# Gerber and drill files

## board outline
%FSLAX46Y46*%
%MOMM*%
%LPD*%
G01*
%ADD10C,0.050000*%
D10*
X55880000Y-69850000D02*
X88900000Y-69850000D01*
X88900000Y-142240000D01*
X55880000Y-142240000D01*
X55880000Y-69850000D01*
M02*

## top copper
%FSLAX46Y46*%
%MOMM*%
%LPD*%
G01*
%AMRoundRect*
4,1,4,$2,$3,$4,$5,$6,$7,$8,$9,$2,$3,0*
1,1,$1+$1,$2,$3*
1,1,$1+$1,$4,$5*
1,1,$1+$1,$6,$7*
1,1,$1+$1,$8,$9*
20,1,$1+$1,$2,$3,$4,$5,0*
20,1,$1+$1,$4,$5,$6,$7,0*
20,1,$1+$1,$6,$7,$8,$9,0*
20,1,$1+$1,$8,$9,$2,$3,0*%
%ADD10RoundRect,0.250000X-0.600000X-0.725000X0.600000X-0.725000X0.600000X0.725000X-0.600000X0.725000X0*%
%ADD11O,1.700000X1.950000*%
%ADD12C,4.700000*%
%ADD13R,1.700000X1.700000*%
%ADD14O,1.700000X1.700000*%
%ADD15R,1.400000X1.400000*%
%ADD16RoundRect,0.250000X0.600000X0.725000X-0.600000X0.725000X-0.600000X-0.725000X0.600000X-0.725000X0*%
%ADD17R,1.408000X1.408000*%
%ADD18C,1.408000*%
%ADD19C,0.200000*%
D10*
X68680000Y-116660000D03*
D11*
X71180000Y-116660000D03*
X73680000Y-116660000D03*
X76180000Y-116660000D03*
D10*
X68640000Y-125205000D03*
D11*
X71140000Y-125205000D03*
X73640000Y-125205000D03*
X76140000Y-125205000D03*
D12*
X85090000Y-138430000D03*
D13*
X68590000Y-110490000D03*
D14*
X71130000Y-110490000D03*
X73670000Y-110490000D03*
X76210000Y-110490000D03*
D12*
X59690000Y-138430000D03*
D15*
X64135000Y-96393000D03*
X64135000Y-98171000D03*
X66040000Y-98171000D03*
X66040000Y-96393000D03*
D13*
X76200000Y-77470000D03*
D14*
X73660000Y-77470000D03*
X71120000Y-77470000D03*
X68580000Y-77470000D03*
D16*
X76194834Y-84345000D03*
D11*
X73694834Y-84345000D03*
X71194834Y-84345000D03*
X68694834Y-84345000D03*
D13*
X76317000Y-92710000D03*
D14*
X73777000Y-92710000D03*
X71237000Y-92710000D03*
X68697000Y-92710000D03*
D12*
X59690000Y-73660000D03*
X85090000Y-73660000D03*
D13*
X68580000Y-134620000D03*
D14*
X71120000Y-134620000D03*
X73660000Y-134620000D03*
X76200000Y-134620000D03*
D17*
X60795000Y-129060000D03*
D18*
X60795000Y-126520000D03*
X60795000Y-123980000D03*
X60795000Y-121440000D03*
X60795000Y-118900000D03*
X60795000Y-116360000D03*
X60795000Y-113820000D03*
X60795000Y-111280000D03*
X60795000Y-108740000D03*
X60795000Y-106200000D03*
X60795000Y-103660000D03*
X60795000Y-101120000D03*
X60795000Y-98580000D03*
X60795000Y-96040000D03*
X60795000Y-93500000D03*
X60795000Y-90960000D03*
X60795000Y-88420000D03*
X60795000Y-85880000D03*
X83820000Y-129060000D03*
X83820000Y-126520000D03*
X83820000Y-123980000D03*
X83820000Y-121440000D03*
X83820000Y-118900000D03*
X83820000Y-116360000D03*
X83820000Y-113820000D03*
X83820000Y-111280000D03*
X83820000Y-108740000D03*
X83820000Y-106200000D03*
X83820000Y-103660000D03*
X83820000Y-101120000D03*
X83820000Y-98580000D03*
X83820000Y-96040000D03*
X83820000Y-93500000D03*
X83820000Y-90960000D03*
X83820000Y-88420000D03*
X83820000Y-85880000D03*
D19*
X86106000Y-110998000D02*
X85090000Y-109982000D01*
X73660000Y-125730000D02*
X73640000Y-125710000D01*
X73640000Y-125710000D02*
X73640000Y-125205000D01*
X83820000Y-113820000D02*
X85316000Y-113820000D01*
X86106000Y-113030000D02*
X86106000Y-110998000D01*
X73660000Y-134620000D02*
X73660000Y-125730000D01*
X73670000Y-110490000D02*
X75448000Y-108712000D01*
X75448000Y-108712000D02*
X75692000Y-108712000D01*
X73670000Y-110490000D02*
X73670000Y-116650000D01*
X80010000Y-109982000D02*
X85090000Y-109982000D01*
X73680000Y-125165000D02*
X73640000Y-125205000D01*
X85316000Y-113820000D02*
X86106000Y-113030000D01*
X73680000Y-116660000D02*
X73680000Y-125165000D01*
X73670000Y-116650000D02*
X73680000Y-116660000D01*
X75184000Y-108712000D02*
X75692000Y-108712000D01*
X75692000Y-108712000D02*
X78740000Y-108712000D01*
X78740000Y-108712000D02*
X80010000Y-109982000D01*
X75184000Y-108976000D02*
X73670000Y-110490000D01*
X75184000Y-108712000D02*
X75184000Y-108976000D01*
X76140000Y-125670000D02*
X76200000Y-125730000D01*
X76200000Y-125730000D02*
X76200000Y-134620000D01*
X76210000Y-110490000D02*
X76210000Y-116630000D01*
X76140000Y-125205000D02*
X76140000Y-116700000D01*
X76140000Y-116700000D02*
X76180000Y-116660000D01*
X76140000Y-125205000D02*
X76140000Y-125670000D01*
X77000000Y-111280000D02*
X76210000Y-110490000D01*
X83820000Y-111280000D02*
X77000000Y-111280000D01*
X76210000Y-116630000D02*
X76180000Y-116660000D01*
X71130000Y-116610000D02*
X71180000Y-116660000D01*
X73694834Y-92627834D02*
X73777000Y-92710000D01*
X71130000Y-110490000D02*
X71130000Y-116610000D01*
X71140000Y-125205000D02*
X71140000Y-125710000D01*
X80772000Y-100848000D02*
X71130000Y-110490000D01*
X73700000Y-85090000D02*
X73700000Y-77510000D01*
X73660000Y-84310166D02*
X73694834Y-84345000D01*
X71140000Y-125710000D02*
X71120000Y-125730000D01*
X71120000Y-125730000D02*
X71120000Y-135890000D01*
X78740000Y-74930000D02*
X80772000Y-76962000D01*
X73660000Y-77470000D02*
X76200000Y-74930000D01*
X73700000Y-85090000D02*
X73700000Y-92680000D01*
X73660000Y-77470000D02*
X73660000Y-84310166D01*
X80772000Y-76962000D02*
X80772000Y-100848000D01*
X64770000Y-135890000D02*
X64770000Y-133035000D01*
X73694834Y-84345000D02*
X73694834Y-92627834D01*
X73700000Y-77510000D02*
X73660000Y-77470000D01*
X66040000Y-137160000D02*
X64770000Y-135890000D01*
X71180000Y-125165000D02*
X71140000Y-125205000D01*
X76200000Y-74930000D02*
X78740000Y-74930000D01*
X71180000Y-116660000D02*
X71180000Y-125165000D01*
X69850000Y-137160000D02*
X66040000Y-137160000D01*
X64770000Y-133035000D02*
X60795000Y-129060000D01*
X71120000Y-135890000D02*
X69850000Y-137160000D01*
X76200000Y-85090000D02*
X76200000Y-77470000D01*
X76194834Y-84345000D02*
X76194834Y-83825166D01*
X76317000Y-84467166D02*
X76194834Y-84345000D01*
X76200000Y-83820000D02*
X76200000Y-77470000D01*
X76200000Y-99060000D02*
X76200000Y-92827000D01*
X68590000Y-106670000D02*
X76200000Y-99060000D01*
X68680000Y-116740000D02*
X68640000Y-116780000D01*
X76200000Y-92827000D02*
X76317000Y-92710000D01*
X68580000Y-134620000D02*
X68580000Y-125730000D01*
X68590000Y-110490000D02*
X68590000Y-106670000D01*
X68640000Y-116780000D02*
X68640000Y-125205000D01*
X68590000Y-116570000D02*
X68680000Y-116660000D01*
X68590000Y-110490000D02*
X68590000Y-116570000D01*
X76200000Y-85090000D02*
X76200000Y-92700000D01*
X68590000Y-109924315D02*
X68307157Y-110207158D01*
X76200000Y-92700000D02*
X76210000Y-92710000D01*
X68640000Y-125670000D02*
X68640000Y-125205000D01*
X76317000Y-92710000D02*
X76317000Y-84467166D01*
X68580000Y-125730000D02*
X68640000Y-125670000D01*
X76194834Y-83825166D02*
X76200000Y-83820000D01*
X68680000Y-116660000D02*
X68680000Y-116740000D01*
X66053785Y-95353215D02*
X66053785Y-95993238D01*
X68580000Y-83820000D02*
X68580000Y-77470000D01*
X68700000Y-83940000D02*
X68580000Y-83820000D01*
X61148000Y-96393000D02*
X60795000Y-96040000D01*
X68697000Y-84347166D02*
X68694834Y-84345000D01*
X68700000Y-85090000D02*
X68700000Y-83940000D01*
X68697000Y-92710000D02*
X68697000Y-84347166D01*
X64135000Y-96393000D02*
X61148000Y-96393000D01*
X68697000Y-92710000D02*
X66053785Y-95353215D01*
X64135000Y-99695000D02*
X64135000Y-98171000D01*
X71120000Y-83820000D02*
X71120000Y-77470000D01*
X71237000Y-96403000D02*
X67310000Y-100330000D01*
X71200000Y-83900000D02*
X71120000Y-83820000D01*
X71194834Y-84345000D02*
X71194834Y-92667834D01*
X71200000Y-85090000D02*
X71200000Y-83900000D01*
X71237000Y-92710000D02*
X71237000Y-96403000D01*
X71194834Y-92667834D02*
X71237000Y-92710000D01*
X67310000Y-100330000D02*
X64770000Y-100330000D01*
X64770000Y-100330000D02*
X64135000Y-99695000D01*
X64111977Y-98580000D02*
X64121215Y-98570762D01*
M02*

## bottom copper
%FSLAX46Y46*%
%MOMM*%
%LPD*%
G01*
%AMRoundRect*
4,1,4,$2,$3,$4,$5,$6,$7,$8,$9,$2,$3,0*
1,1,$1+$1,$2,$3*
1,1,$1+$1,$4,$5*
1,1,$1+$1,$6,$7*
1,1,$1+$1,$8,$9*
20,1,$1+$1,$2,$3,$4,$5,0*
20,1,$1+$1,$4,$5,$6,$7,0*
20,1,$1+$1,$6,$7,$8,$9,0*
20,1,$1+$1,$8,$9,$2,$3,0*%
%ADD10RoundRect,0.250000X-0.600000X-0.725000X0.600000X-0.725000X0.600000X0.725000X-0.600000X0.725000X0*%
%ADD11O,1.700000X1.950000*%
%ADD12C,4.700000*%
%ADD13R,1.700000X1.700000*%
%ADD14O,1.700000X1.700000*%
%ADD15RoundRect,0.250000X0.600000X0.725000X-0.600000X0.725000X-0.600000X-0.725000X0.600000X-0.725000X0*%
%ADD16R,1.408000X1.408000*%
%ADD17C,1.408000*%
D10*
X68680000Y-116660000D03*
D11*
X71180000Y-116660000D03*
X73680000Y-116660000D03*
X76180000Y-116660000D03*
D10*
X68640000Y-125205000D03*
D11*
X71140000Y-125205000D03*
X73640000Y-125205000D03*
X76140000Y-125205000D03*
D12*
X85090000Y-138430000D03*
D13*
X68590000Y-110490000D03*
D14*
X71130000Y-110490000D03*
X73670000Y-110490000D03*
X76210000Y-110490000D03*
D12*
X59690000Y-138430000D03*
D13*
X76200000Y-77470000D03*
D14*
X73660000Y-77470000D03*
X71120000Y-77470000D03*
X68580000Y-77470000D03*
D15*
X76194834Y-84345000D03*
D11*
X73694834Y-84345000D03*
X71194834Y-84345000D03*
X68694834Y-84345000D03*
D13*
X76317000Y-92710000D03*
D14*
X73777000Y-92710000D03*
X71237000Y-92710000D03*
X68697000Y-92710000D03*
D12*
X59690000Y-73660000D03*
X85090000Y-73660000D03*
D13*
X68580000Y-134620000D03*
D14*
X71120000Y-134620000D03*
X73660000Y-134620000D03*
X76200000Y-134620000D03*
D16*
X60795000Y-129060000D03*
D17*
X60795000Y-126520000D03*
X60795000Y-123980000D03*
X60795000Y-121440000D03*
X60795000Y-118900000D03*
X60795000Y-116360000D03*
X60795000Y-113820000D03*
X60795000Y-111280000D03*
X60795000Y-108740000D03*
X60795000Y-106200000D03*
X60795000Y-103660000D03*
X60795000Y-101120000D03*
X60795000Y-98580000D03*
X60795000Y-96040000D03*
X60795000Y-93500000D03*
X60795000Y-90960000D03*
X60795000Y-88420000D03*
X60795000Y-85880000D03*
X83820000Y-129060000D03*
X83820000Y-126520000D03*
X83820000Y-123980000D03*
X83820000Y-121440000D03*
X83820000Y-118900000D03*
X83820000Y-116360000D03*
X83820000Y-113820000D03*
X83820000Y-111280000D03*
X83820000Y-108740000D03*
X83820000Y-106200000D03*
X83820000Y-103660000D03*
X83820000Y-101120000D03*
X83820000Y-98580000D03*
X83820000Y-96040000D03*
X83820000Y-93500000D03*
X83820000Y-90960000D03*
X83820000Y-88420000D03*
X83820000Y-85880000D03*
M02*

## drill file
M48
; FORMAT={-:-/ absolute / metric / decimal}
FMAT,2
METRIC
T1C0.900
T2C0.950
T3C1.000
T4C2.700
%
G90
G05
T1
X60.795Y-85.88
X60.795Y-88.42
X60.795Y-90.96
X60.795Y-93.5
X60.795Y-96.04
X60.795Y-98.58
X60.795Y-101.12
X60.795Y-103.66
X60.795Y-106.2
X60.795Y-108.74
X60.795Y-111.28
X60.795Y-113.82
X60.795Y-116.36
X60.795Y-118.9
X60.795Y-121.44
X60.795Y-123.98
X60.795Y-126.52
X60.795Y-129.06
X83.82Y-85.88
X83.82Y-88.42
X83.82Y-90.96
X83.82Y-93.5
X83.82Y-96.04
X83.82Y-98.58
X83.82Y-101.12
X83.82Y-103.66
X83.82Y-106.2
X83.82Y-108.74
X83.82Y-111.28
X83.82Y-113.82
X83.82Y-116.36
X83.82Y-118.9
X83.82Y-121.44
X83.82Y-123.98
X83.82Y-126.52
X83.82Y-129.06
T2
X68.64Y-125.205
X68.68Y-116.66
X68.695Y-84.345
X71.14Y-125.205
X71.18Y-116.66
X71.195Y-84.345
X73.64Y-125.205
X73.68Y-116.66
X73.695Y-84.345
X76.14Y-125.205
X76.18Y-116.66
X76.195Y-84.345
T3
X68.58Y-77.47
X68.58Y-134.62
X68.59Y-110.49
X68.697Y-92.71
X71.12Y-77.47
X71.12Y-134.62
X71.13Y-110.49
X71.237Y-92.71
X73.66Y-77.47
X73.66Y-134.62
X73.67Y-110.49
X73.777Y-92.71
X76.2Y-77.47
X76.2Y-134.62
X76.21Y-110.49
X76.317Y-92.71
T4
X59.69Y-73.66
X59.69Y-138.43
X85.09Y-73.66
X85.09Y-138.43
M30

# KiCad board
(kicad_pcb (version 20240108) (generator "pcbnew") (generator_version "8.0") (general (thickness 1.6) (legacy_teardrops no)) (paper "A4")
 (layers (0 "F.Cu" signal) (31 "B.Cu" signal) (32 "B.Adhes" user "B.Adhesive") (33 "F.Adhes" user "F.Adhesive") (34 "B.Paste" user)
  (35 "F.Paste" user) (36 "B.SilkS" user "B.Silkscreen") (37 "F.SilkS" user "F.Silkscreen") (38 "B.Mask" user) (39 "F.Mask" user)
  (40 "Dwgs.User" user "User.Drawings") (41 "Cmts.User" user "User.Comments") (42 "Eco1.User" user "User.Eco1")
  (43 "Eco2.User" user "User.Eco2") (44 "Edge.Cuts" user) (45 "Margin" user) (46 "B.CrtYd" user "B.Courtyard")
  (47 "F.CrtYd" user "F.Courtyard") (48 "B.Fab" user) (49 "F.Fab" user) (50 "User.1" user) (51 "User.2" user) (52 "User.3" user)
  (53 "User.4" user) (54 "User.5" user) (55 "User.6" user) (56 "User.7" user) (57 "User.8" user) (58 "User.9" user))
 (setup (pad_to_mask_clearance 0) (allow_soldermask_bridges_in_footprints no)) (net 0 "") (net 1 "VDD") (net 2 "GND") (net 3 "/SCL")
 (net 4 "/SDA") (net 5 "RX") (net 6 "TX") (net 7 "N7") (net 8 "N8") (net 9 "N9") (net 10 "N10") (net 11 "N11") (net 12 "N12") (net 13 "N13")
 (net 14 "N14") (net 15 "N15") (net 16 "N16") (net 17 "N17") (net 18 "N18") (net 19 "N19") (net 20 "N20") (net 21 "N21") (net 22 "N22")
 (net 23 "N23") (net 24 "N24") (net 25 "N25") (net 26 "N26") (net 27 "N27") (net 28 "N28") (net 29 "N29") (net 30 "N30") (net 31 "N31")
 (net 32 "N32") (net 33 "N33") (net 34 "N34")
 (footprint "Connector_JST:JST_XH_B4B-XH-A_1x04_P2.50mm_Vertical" (layer "F.Cu") (at 68.68 116.66)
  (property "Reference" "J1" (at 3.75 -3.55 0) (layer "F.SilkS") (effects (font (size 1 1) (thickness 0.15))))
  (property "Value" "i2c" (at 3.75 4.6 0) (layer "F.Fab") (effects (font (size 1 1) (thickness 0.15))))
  (pad "1" thru_hole roundrect (at 0 0) (size 1.7 1.95) (drill 0.95) (layers "*.Cu" "*.Mask") (remove_unused_layers no)
   (roundrect_rratio 0.147059) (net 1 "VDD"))
  (pad "2" thru_hole oval (at 2.5 0) (size 1.7 1.95) (drill 0.95) (layers "*.Cu" "*.Mask") (remove_unused_layers no) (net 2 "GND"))
  (pad "3" thru_hole oval (at 5 0) (size 1.7 1.95) (drill 0.95) (layers "*.Cu" "*.Mask") (remove_unused_layers no) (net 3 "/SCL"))
  (pad "4" thru_hole oval (at 7.5 0) (size 1.7 1.95) (drill 0.95) (layers "*.Cu" "*.Mask") (remove_unused_layers no) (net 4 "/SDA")))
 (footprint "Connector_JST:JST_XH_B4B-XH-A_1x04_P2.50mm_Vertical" (layer "F.Cu") (at 68.64 125.205)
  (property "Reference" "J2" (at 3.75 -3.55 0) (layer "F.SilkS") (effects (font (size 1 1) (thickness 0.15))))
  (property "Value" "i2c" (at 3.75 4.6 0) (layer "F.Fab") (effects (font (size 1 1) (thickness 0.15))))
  (pad "1" thru_hole roundrect (at 0 0) (size 1.7 1.95) (drill 0.95) (layers "*.Cu" "*.Mask") (remove_unused_layers no)
   (roundrect_rratio 0.147059) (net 1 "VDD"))
  (pad "2" thru_hole oval (at 2.5 0) (size 1.7 1.95) (drill 0.95) (layers "*.Cu" "*.Mask") (remove_unused_layers no) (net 2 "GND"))
  (pad "3" thru_hole oval (at 5 0) (size 1.7 1.95) (drill 0.95) (layers "*.Cu" "*.Mask") (remove_unused_layers no) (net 3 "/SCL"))
  (pad "4" thru_hole oval (at 7.5 0) (size 1.7 1.95) (drill 0.95) (layers "*.Cu" "*.Mask") (remove_unused_layers no) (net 4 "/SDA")))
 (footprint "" (layer "F.Cu") (at 85.09 138.43)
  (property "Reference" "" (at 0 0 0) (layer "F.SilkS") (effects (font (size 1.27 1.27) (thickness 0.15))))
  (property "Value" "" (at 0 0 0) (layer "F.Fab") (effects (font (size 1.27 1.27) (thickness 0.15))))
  (pad "1" thru_hole circle (at 0 0) (size 4.7 4.7) (drill 2.7) (layers "*.Cu" "*.Mask") (remove_unused_layers no)))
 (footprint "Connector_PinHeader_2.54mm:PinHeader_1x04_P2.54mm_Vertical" (layer "F.Cu") (at 68.59 110.49 90)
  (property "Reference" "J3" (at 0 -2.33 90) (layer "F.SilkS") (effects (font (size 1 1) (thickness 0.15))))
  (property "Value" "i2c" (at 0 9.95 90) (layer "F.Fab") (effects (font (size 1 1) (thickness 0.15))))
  (pad "1" thru_hole rect (at 0 0 90) (size 1.7 1.7) (drill 1) (layers "*.Cu" "*.Mask") (remove_unused_layers no) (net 1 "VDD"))
  (pad "2" thru_hole oval (at 0 2.54 90) (size 1.7 1.7) (drill 1) (layers "*.Cu" "*.Mask") (remove_unused_layers no) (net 2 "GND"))
  (pad "3" thru_hole oval (at 0 5.08 90) (size 1.7 1.7) (drill 1) (layers "*.Cu" "*.Mask") (remove_unused_layers no) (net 3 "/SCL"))
  (pad "4" thru_hole oval (at 0 7.62 90) (size 1.7 1.7) (drill 1) (layers "*.Cu" "*.Mask") (remove_unused_layers no) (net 4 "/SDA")))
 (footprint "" (layer "F.Cu") (at 59.69 138.43)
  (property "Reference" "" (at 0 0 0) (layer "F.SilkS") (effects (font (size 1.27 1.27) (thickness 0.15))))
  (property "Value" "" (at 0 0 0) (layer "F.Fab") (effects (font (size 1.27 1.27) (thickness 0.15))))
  (pad "1" thru_hole circle (at 0 0) (size 4.7 4.7) (drill 2.7) (layers "*.Cu" "*.Mask") (remove_unused_layers no)))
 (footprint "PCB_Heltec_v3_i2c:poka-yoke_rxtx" (layer "F.Cu") (at 65.024 94.742)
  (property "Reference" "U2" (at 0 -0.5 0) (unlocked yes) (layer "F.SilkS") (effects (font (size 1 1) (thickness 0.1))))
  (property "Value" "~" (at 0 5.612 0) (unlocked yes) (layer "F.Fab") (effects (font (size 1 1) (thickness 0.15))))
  (pad "1" smd rect (at -0.889 1.651) (size 1.4 1.4) (layers "F.Cu" "F.Paste" "F.Mask") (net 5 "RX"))
  (pad "2" smd rect (at -0.889 3.429) (size 1.4 1.4) (layers "F.Cu" "F.Paste" "F.Mask") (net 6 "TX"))
  (pad "3" smd rect (at 1.016 3.429) (size 1.4 1.4) (layers "F.Cu" "F.Paste" "F.Mask") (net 6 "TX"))
  (pad "4" smd rect (at 1.016 1.651) (size 1.4 1.4) (layers "F.Cu" "F.Paste" "F.Mask") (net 5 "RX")))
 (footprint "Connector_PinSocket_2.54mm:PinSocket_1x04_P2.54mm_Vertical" (layer "F.Cu") (at 76.2 77.47 -90)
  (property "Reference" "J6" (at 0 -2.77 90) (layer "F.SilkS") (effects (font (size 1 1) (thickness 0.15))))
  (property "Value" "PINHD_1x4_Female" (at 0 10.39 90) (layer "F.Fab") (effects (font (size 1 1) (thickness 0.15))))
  (pad "1" thru_hole rect (at 0 0 270) (size 1.7 1.7) (drill 1) (layers "*.Cu" "*.Mask") (remove_unused_layers no) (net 1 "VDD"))
  (pad "2" thru_hole oval (at 0 2.54 270) (size 1.7 1.7) (drill 1) (layers "*.Cu" "*.Mask") (remove_unused_layers no) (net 2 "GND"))
  (pad "3" thru_hole oval (at 0 5.08 270) (size 1.7 1.7) (drill 1) (layers "*.Cu" "*.Mask") (remove_unused_layers no) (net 6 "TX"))
  (pad "4" thru_hole oval (at 0 7.62 270) (size 1.7 1.7) (drill 1) (layers "*.Cu" "*.Mask") (remove_unused_layers no) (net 5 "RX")))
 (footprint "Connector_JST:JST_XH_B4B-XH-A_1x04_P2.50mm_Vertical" (layer "F.Cu") (at 76.194834 84.345 180)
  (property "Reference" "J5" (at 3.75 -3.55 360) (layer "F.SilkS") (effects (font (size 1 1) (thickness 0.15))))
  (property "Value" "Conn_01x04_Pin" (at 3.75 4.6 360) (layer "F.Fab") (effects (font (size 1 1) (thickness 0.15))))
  (pad "1" thru_hole roundrect (at 0 0 180) (size 1.7 1.95) (drill 0.95) (layers "*.Cu" "*.Mask") (remove_unused_layers no)
   (roundrect_rratio 0.147059) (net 1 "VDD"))
  (pad "2" thru_hole oval (at 2.5 0 180) (size 1.7 1.95) (drill 0.95) (layers "*.Cu" "*.Mask") (remove_unused_layers no) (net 2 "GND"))
  (pad "3" thru_hole oval (at 5 0 180) (size 1.7 1.95) (drill 0.95) (layers "*.Cu" "*.Mask") (remove_unused_layers no) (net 6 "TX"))
  (pad "4" thru_hole oval (at 7.5 0 180) (size 1.7 1.95) (drill 0.95) (layers "*.Cu" "*.Mask") (remove_unused_layers no) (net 5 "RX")))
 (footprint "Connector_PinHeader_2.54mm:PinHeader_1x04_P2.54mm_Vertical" (layer "F.Cu") (at 76.317 92.71 -90)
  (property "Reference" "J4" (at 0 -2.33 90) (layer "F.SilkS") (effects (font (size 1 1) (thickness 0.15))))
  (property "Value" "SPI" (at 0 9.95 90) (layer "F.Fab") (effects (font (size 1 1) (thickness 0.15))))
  (pad "1" thru_hole rect (at 0 0 270) (size 1.7 1.7) (drill 1) (layers "*.Cu" "*.Mask") (remove_unused_layers no) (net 1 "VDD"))
  (pad "2" thru_hole oval (at 0 2.54 270) (size 1.7 1.7) (drill 1) (layers "*.Cu" "*.Mask") (remove_unused_layers no) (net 2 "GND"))
  (pad "3" thru_hole oval (at 0 5.08 270) (size 1.7 1.7) (drill 1) (layers "*.Cu" "*.Mask") (remove_unused_layers no) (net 6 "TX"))
  (pad "4" thru_hole oval (at 0 7.62 270) (size 1.7 1.7) (drill 1) (layers "*.Cu" "*.Mask") (remove_unused_layers no) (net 5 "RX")))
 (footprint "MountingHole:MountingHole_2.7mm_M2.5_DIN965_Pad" (layer "F.Cu") (at 59.69 73.66)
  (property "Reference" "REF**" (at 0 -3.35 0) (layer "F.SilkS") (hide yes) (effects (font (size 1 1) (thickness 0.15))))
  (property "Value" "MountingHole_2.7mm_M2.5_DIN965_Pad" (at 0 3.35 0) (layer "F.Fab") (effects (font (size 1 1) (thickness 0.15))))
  (pad "1" thru_hole circle (at 0 0) (size 4.7 4.7) (drill 2.7) (layers "*.Cu" "*.Mask") (remove_unused_layers no)))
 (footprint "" (layer "F.Cu") (at 85.09 73.66)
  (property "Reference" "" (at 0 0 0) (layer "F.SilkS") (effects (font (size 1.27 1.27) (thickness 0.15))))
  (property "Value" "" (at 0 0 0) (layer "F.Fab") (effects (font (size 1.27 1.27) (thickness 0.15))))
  (pad "1" thru_hole circle (at 0 0) (size 4.7 4.7) (drill 2.7) (layers "*.Cu" "*.Mask") (remove_unused_layers no)))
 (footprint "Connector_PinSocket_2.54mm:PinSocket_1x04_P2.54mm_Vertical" (layer "F.Cu") (at 68.58 134.62 90)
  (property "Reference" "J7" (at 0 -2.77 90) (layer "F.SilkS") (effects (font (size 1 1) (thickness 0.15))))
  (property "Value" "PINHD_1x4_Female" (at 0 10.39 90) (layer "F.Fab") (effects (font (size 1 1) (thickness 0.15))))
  (pad "1" thru_hole rect (at 0 0 90) (size 1.7 1.7) (drill 1) (layers "*.Cu" "*.Mask") (remove_unused_layers no) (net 1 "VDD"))
  (pad "2" thru_hole oval (at 0 2.54 90) (size 1.7 1.7) (drill 1) (layers "*.Cu" "*.Mask") (remove_unused_layers no) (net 2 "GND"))
  (pad "3" thru_hole oval (at 0 5.08 90) (size 1.7 1.7) (drill 1) (layers "*.Cu" "*.Mask") (remove_unused_layers no) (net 3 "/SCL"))
  (pad "4" thru_hole oval (at 0 7.62 90) (size 1.7 1.7) (drill 1) (layers "*.Cu" "*.Mask") (remove_unused_layers no) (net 4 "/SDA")))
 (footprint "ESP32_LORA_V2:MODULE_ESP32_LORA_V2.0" (layer "B.Cu") (at 72.3075 106.68 90)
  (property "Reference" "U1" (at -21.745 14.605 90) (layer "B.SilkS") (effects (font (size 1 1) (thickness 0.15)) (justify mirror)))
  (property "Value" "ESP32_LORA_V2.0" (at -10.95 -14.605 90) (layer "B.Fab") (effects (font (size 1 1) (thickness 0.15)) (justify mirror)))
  (pad "J2_1" thru_hole rect (at -22.38 -11.5125 90) (size 1.408 1.408) (drill 0.9) (layers "*.Cu" "*.Mask") (remove_unused_layers no)
   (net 2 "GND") (solder_mask_margin 0.102))
  (pad "J2_2" thru_hole circle (at -19.84 -11.5125 90) (size 1.408 1.408) (drill 0.9) (layers "*.Cu" "*.Mask") (remove_unused_layers no)
   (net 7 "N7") (solder_mask_margin 0.102))
  (pad "J2_3" thru_hole circle (at -17.3 -11.5125 90) (size 1.408 1.408) (drill 0.9) (layers "*.Cu" "*.Mask") (remove_unused_layers no)
   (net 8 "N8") (solder_mask_margin 0.102))
  (pad "J2_4" thru_hole circle (at -14.76 -11.5125 90) (size 1.408 1.408) (drill 0.9) (layers "*.Cu" "*.Mask") (remove_unused_layers no)
   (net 8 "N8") (solder_mask_margin 0.102))
  (pad "J2_5" thru_hole circle (at -12.22 -11.5125 90) (size 1.408 1.408) (drill 0.9) (layers "*.Cu" "*.Mask") (remove_unused_layers no)
   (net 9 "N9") (solder_mask_margin 0.102))
  (pad "J2_6" thru_hole circle (at -9.68 -11.5125 90) (size 1.408 1.408) (drill 0.9) (layers "*.Cu" "*.Mask") (remove_unused_layers no)
   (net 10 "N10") (solder_mask_margin 0.102))
  (pad "J2_7" thru_hole circle (at -7.14 -11.5125 90) (size 1.408 1.408) (drill 0.9) (layers "*.Cu" "*.Mask") (remove_unused_layers no)
   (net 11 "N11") (solder_mask_margin 0.102))
  (pad "J2_8" thru_hole circle (at -4.6 -11.5125 90) (size 1.408 1.408) (drill 0.9) (layers "*.Cu" "*.Mask") (remove_unused_layers no)
   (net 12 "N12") (solder_mask_margin 0.102))
  (pad "J2_9" thru_hole circle (at -2.06 -11.5125 90) (size 1.408 1.408) (drill 0.9) (layers "*.Cu" "*.Mask") (remove_unused_layers no)
   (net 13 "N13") (solder_mask_margin 0.102))
  (pad "J2_10" thru_hole circle (at 0.48 -11.5125 90) (size 1.408 1.408) (drill 0.9) (layers "*.Cu" "*.Mask") (remove_unused_layers no)
   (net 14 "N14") (solder_mask_margin 0.102))
  (pad "J2_11" thru_hole circle (at 3.02 -11.5125 90) (size 1.408 1.408) (drill 0.9) (layers "*.Cu" "*.Mask") (remove_unused_layers no)
   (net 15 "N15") (solder_mask_margin 0.102))
  (pad "J2_12" thru_hole circle (at 5.56 -11.5125 90) (size 1.408 1.408) (drill 0.9) (layers "*.Cu" "*.Mask") (remove_unused_layers no)
   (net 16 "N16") (solder_mask_margin 0.102))
  (pad "J2_13" thru_hole circle (at 8.1 -11.5125 90) (size 1.408 1.408) (drill 0.9) (layers "*.Cu" "*.Mask") (remove_unused_layers no)
   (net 6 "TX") (solder_mask_margin 0.102))
  (pad "J2_14" thru_hole circle (at 10.64 -11.5125 90) (size 1.408 1.408) (drill 0.9) (layers "*.Cu" "*.Mask") (remove_unused_layers no)
   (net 5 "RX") (solder_mask_margin 0.102))
  (pad "J2_15" thru_hole circle (at 13.18 -11.5125 90) (size 1.408 1.408) (drill 0.9) (layers "*.Cu" "*.Mask") (remove_unused_layers no)
   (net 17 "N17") (solder_mask_margin 0.102))
  (pad "J2_16" thru_hole circle (at 15.72 -11.5125 90) (size 1.408 1.408) (drill 0.9) (layers "*.Cu" "*.Mask") (remove_unused_layers no)
   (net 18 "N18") (solder_mask_margin 0.102))
  (pad "J2_17" thru_hole circle (at 18.26 -11.5125 90) (size 1.408 1.408) (drill 0.9) (layers "*.Cu" "*.Mask") (remove_unused_layers no)
   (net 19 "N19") (solder_mask_margin 0.102))
  (pad "J2_18" thru_hole circle (at 20.8 -11.5125 90) (size 1.408 1.408) (drill 0.9) (layers "*.Cu" "*.Mask") (remove_unused_layers no)
   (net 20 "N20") (solder_mask_margin 0.102))
  (pad "J3_1" thru_hole circle (at -22.38 11.5125 90) (size 1.408 1.408) (drill 0.9) (layers "*.Cu" "*.Mask") (remove_unused_layers no)
   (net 2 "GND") (solder_mask_margin 0.102))
  (pad "J3_2" thru_hole circle (at -19.84 11.5125 90) (size 1.408 1.408) (drill 0.9) (layers "*.Cu" "*.Mask") (remove_unused_layers no)
   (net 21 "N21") (solder_mask_margin 0.102))
  (pad "J3_3" thru_hole circle (at -17.3 11.5125 90) (size 1.408 1.408) (drill 0.9) (layers "*.Cu" "*.Mask") (remove_unused_layers no)
   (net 21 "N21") (solder_mask_margin 0.102))
  (pad "J3_4" thru_hole circle (at -14.76 11.5125 90) (size 1.408 1.408) (drill 0.9) (layers "*.Cu" "*.Mask") (remove_unused_layers no)
   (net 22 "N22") (solder_mask_margin 0.102))
  (pad "J3_5" thru_hole circle (at -12.22 11.5125 90) (size 1.408 1.408) (drill 0.9) (layers "*.Cu" "*.Mask") (remove_unused_layers no)
   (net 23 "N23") (solder_mask_margin 0.102))
  (pad "J3_6" thru_hole circle (at -9.68 11.5125 90) (size 1.408 1.408) (drill 0.9) (layers "*.Cu" "*.Mask") (remove_unused_layers no)
   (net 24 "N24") (solder_mask_margin 0.102))
  (pad "J3_7" thru_hole circle (at -7.14 11.5125 90) (size 1.408 1.408) (drill 0.9) (layers "*.Cu" "*.Mask") (remove_unused_layers no)
   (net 3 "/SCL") (solder_mask_margin 0.102))
  (pad "J3_8" thru_hole circle (at -4.6 11.5125 90) (size 1.408 1.408) (drill 0.9) (layers "*.Cu" "*.Mask") (remove_unused_layers no)
   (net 4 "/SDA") (solder_mask_margin 0.102))
  (pad "J3_9" thru_hole circle (at -2.06 11.5125 90) (size 1.408 1.408) (drill 0.9) (layers "*.Cu" "*.Mask") (remove_unused_layers no)
   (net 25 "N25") (solder_mask_margin 0.102))
  (pad "J3_10" thru_hole circle (at 0.48 11.5125 90) (size 1.408 1.408) (drill 0.9) (layers "*.Cu" "*.Mask") (remove_unused_layers no)
   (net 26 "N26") (solder_mask_margin 0.102))
  (pad "J3_11" thru_hole circle (at 3.02 11.5125 90) (size 1.408 1.408) (drill 0.9) (layers "*.Cu" "*.Mask") (remove_unused_layers no)
   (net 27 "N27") (solder_mask_margin 0.102))
  (pad "J3_12" thru_hole circle (at 5.56 11.5125 90) (size 1.408 1.408) (drill 0.9) (layers "*.Cu" "*.Mask") (remove_unused_layers no)
   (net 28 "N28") (solder_mask_margin 0.102))
  (pad "J3_13" thru_hole circle (at 8.1 11.5125 90) (size 1.408 1.408) (drill 0.9) (layers "*.Cu" "*.Mask") (remove_unused_layers no)
   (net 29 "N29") (solder_mask_margin 0.102))
  (pad "J3_14" thru_hole circle (at 10.64 11.5125 90) (size 1.408 1.408) (drill 0.9) (layers "*.Cu" "*.Mask") (remove_unused_layers no)
   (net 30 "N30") (solder_mask_margin 0.102))
  (pad "J3_15" thru_hole circle (at 13.18 11.5125 90) (size 1.408 1.408) (drill 0.9) (layers "*.Cu" "*.Mask") (remove_unused_layers no)
   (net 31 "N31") (solder_mask_margin 0.102))
  (pad "J3_16" thru_hole circle (at 15.72 11.5125 90) (size 1.408 1.408) (drill 0.9) (layers "*.Cu" "*.Mask") (remove_unused_layers no)
   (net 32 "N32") (solder_mask_margin 0.102))
  (pad "J3_17" thru_hole circle (at 18.26 11.5125 90) (size 1.408 1.408) (drill 0.9) (layers "*.Cu" "*.Mask") (remove_unused_layers no)
   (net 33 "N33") (solder_mask_margin 0.102))
  (pad "J3_18" thru_hole circle (at 20.8 11.5125 90) (size 1.408 1.408) (drill 0.9) (layers "*.Cu" "*.Mask") (remove_unused_layers no)
   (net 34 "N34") (solder_mask_margin 0.102)))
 (gr_rect (start 55.88 69.85) (end 88.9 142.24) (stroke (width 0.05) (type default)) (fill none) (layer "Edge.Cuts"))
 (segment (start 86.106 110.998) (end 85.09 109.982) (width 0.2) (layer "F.Cu") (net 3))
 (segment (start 73.66 125.73) (end 73.64 125.71) (width 0.2) (layer "F.Cu") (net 3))
 (segment (start 73.64 125.71) (end 73.64 125.205) (width 0.2) (layer "F.Cu") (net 3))
 (segment (start 83.82 113.82) (end 85.316 113.82) (width 0.2) (layer "F.Cu") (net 3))
 (segment (start 86.106 113.03) (end 86.106 110.998) (width 0.2) (layer "F.Cu") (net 3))
 (segment (start 73.66 134.62) (end 73.66 125.73) (width 0.2) (layer "F.Cu") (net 3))
 (segment (start 73.67 110.49) (end 75.448 108.712) (width 0.2) (layer "F.Cu") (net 3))
 (segment (start 75.448 108.712) (end 75.692 108.712) (width 0.2) (layer "F.Cu") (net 3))
 (segment (start 73.67 110.49) (end 73.67 116.65) (width 0.2) (layer "F.Cu") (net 3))
 (segment (start 80.01 109.982) (end 85.09 109.982) (width 0.2) (layer "F.Cu") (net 3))
 (segment (start 73.68 125.165) (end 73.64 125.205) (width 0.2) (layer "F.Cu") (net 3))
 (segment (start 85.316 113.82) (end 86.106 113.03) (width 0.2) (layer "F.Cu") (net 3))
 (segment (start 73.68 116.66) (end 73.68 125.165) (width 0.2) (layer "F.Cu") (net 3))
 (segment (start 73.67 116.65) (end 73.68 116.66) (width 0.2) (layer "F.Cu") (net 3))
 (segment (start 75.184 108.712) (end 75.692 108.712) (width 0.2) (layer "F.Cu") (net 3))
 (segment (start 75.692 108.712) (end 78.74 108.712) (width 0.2) (layer "F.Cu") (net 3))
 (segment (start 78.74 108.712) (end 80.01 109.982) (width 0.2) (layer "F.Cu") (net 3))
 (segment (start 75.184 108.976) (end 73.67 110.49) (width 0.2) (layer "F.Cu") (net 3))
 (segment (start 75.184 108.712) (end 75.184 108.976) (width 0.2) (layer "F.Cu") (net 3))
 (segment (start 76.14 125.67) (end 76.2 125.73) (width 0.2) (layer "F.Cu") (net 4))
 (segment (start 76.2 125.73) (end 76.2 134.62) (width 0.2) (layer "F.Cu") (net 4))
 (segment (start 76.21 110.49) (end 76.21 116.63) (width 0.2) (layer "F.Cu") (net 4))
 (segment (start 76.14 125.205) (end 76.14 116.7) (width 0.2) (layer "F.Cu") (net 4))
 (segment (start 76.14 116.7) (end 76.18 116.66) (width 0.2) (layer "F.Cu") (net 4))
 (segment (start 76.14 125.205) (end 76.14 125.67) (width 0.2) (layer "F.Cu") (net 4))
 (segment (start 77 111.28) (end 76.21 110.49) (width 0.2) (layer "F.Cu") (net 4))
 (segment (start 83.82 111.28) (end 77 111.28) (width 0.2) (layer "F.Cu") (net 4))
 (segment (start 76.21 116.63) (end 76.18 116.66) (width 0.2) (layer "F.Cu") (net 4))
 (segment (start 71.13 116.61) (end 71.18 116.66) (width 0.2) (layer "F.Cu") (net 2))
 (segment (start 73.694834 92.627834) (end 73.777 92.71) (width 0.2) (layer "F.Cu") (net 2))
 (segment (start 71.13 110.49) (end 71.13 116.61) (width 0.2) (layer "F.Cu") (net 2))
 (segment (start 71.14 125.205) (end 71.14 125.71) (width 0.2) (layer "F.Cu") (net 2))
 (segment (start 80.772 100.848) (end 71.13 110.49) (width 0.2) (layer "F.Cu") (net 2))
 (segment (start 73.7 85.09) (end 73.7 77.51) (width 0.2) (layer "F.Cu") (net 2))
 (segment (start 73.66 84.310166) (end 73.694834 84.345) (width 0.2) (layer "F.Cu") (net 2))
 (segment (start 71.14 125.71) (end 71.12 125.73) (width 0.2) (layer "F.Cu") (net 2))
 (segment (start 71.12 125.73) (end 71.12 135.89) (width 0.2) (layer "F.Cu") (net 2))
 (segment (start 78.74 74.93) (end 80.772 76.962) (width 0.2) (layer "F.Cu") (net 2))
 (segment (start 73.66 77.47) (end 76.2 74.93) (width 0.2) (layer "F.Cu") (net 2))
 (segment (start 73.7 85.09) (end 73.7 92.68) (width 0.2) (layer "F.Cu") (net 2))
 (segment (start 73.66 77.47) (end 73.66 84.310166) (width 0.2) (layer "F.Cu") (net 2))
 (segment (start 80.772 76.962) (end 80.772 100.848) (width 0.2) (layer "F.Cu") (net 2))
 (segment (start 64.77 135.89) (end 64.77 133.035) (width 0.2) (layer "F.Cu") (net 2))
 (segment (start 73.694834 84.345) (end 73.694834 92.627834) (width 0.2) (layer "F.Cu") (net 2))
 (segment (start 73.7 77.51) (end 73.66 77.47) (width 0.2) (layer "F.Cu") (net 2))
 (segment (start 66.04 137.16) (end 64.77 135.89) (width 0.2) (layer "F.Cu") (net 2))
 (segment (start 71.18 125.165) (end 71.14 125.205) (width 0.2) (layer "F.Cu") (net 2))
 (segment (start 76.2 74.93) (end 78.74 74.93) (width 0.2) (layer "F.Cu") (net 2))
 (segment (start 71.18 116.66) (end 71.18 125.165) (width 0.2) (layer "F.Cu") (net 2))
 (segment (start 69.85 137.16) (end 66.04 137.16) (width 0.2) (layer "F.Cu") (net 2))
 (segment (start 64.77 133.035) (end 60.795 129.06) (width 0.2) (layer "F.Cu") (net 2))
 (segment (start 71.12 135.89) (end 69.85 137.16) (width 0.2) (layer "F.Cu") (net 2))
 (segment (start 76.2 85.09) (end 76.2 77.47) (width 0.2) (layer "F.Cu") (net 1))
 (segment (start 76.194834 84.345) (end 76.194834 83.825166) (width 0.2) (layer "F.Cu") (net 1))
 (segment (start 76.317 84.467166) (end 76.194834 84.345) (width 0.2) (layer "F.Cu") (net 1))
 (segment (start 76.2 83.82) (end 76.2 77.47) (width 0.2) (layer "F.Cu") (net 1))
 (segment (start 76.2 99.06) (end 76.2 92.827) (width 0.2) (layer "F.Cu") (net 1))
 (segment (start 68.59 106.67) (end 76.2 99.06) (width 0.2) (layer "F.Cu") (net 1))
 (segment (start 68.68 116.74) (end 68.64 116.78) (width 0.2) (layer "F.Cu") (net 1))
 (segment (start 76.2 92.827) (end 76.317 92.71) (width 0.2) (layer "F.Cu") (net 1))
 (segment (start 68.58 134.62) (end 68.58 125.73) (width 0.2) (layer "F.Cu") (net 1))
 (segment (start 68.59 110.49) (end 68.59 106.67) (width 0.2) (layer "F.Cu") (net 1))
 (segment (start 68.64 116.78) (end 68.64 125.205) (width 0.2) (layer "F.Cu") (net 1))
 (segment (start 68.59 116.57) (end 68.68 116.66) (width 0.2) (layer "F.Cu") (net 1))
 (segment (start 68.59 110.49) (end 68.59 116.57) (width 0.2) (layer "F.Cu") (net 1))
 (segment (start 76.2 85.09) (end 76.2 92.7) (width 0.2) (layer "F.Cu") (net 1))
 (segment (start 68.59 109.924315) (end 68.307157 110.207158) (width 0.2) (layer "F.Cu") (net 1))
 (segment (start 76.2 92.7) (end 76.21 92.71) (width 0.2) (layer "F.Cu") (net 1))
 (segment (start 68.64 125.67) (end 68.64 125.205) (width 0.2) (layer "F.Cu") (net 1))
 (segment (start 76.317 92.71) (end 76.317 84.467166) (width 0.2) (layer "F.Cu") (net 1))
 (segment (start 68.58 125.73) (end 68.64 125.67) (width 0.2) (layer "F.Cu") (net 1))
 (segment (start 76.194834 83.825166) (end 76.2 83.82) (width 0.2) (layer "F.Cu") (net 1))
 (segment (start 68.68 116.66) (end 68.68 116.74) (width 0.2) (layer "F.Cu") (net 1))
 (segment (start 66.053785 95.353215) (end 66.053785 95.993238) (width 0.2) (layer "F.Cu") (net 5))
 (segment (start 68.58 83.82) (end 68.58 77.47) (width 0.2) (layer "F.Cu") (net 5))
 (segment (start 68.7 83.94) (end 68.58 83.82) (width 0.2) (layer "F.Cu") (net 5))
 (segment (start 61.148 96.393) (end 60.795 96.04) (width 0.2) (layer "F.Cu") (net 5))
 (segment (start 68.697 84.347166) (end 68.694834 84.345) (width 0.2) (layer "F.Cu") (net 5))
 (segment (start 68.7 85.09) (end 68.7 83.94) (width 0.2) (layer "F.Cu") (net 5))
 (segment (start 68.697 92.71) (end 68.697 84.347166) (width 0.2) (layer "F.Cu") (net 5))
 (segment (start 64.135 96.393) (end 61.148 96.393) (width 0.2) (layer "F.Cu") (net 5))
 (segment (start 68.697 92.71) (end 66.053785 95.353215) (width 0.2) (layer "F.Cu") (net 5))
 (segment (start 64.135 99.695) (end 64.135 98.171) (width 0.2) (layer "F.Cu") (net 6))
 (segment (start 71.12 83.82) (end 71.12 77.47) (width 0.2) (layer "F.Cu") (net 6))
 (segment (start 71.237 96.403) (end 67.31 100.33) (width 0.2) (layer "F.Cu") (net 6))
 (segment (start 71.2 83.9) (end 71.12 83.82) (width 0.2) (layer "F.Cu") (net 6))
 (segment (start 71.194834 84.345) (end 71.194834 92.667834) (width 0.2) (layer "F.Cu") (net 6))
 (segment (start 71.2 85.09) (end 71.2 83.9) (width 0.2) (layer "F.Cu") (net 6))
 (segment (start 71.237 92.71) (end 71.237 96.403) (width 0.2) (layer "F.Cu") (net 6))
 (segment (start 71.194834 92.667834) (end 71.237 92.71) (width 0.2) (layer "F.Cu") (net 6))
 (segment (start 67.31 100.33) (end 64.77 100.33) (width 0.2) (layer "F.Cu") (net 6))
 (segment (start 64.77 100.33) (end 64.135 99.695) (width 0.2) (layer "F.Cu") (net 6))
 (segment (start 64.111977 98.58) (end 64.121215 98.570762) (width 0.2) (layer "F.Cu") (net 6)))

